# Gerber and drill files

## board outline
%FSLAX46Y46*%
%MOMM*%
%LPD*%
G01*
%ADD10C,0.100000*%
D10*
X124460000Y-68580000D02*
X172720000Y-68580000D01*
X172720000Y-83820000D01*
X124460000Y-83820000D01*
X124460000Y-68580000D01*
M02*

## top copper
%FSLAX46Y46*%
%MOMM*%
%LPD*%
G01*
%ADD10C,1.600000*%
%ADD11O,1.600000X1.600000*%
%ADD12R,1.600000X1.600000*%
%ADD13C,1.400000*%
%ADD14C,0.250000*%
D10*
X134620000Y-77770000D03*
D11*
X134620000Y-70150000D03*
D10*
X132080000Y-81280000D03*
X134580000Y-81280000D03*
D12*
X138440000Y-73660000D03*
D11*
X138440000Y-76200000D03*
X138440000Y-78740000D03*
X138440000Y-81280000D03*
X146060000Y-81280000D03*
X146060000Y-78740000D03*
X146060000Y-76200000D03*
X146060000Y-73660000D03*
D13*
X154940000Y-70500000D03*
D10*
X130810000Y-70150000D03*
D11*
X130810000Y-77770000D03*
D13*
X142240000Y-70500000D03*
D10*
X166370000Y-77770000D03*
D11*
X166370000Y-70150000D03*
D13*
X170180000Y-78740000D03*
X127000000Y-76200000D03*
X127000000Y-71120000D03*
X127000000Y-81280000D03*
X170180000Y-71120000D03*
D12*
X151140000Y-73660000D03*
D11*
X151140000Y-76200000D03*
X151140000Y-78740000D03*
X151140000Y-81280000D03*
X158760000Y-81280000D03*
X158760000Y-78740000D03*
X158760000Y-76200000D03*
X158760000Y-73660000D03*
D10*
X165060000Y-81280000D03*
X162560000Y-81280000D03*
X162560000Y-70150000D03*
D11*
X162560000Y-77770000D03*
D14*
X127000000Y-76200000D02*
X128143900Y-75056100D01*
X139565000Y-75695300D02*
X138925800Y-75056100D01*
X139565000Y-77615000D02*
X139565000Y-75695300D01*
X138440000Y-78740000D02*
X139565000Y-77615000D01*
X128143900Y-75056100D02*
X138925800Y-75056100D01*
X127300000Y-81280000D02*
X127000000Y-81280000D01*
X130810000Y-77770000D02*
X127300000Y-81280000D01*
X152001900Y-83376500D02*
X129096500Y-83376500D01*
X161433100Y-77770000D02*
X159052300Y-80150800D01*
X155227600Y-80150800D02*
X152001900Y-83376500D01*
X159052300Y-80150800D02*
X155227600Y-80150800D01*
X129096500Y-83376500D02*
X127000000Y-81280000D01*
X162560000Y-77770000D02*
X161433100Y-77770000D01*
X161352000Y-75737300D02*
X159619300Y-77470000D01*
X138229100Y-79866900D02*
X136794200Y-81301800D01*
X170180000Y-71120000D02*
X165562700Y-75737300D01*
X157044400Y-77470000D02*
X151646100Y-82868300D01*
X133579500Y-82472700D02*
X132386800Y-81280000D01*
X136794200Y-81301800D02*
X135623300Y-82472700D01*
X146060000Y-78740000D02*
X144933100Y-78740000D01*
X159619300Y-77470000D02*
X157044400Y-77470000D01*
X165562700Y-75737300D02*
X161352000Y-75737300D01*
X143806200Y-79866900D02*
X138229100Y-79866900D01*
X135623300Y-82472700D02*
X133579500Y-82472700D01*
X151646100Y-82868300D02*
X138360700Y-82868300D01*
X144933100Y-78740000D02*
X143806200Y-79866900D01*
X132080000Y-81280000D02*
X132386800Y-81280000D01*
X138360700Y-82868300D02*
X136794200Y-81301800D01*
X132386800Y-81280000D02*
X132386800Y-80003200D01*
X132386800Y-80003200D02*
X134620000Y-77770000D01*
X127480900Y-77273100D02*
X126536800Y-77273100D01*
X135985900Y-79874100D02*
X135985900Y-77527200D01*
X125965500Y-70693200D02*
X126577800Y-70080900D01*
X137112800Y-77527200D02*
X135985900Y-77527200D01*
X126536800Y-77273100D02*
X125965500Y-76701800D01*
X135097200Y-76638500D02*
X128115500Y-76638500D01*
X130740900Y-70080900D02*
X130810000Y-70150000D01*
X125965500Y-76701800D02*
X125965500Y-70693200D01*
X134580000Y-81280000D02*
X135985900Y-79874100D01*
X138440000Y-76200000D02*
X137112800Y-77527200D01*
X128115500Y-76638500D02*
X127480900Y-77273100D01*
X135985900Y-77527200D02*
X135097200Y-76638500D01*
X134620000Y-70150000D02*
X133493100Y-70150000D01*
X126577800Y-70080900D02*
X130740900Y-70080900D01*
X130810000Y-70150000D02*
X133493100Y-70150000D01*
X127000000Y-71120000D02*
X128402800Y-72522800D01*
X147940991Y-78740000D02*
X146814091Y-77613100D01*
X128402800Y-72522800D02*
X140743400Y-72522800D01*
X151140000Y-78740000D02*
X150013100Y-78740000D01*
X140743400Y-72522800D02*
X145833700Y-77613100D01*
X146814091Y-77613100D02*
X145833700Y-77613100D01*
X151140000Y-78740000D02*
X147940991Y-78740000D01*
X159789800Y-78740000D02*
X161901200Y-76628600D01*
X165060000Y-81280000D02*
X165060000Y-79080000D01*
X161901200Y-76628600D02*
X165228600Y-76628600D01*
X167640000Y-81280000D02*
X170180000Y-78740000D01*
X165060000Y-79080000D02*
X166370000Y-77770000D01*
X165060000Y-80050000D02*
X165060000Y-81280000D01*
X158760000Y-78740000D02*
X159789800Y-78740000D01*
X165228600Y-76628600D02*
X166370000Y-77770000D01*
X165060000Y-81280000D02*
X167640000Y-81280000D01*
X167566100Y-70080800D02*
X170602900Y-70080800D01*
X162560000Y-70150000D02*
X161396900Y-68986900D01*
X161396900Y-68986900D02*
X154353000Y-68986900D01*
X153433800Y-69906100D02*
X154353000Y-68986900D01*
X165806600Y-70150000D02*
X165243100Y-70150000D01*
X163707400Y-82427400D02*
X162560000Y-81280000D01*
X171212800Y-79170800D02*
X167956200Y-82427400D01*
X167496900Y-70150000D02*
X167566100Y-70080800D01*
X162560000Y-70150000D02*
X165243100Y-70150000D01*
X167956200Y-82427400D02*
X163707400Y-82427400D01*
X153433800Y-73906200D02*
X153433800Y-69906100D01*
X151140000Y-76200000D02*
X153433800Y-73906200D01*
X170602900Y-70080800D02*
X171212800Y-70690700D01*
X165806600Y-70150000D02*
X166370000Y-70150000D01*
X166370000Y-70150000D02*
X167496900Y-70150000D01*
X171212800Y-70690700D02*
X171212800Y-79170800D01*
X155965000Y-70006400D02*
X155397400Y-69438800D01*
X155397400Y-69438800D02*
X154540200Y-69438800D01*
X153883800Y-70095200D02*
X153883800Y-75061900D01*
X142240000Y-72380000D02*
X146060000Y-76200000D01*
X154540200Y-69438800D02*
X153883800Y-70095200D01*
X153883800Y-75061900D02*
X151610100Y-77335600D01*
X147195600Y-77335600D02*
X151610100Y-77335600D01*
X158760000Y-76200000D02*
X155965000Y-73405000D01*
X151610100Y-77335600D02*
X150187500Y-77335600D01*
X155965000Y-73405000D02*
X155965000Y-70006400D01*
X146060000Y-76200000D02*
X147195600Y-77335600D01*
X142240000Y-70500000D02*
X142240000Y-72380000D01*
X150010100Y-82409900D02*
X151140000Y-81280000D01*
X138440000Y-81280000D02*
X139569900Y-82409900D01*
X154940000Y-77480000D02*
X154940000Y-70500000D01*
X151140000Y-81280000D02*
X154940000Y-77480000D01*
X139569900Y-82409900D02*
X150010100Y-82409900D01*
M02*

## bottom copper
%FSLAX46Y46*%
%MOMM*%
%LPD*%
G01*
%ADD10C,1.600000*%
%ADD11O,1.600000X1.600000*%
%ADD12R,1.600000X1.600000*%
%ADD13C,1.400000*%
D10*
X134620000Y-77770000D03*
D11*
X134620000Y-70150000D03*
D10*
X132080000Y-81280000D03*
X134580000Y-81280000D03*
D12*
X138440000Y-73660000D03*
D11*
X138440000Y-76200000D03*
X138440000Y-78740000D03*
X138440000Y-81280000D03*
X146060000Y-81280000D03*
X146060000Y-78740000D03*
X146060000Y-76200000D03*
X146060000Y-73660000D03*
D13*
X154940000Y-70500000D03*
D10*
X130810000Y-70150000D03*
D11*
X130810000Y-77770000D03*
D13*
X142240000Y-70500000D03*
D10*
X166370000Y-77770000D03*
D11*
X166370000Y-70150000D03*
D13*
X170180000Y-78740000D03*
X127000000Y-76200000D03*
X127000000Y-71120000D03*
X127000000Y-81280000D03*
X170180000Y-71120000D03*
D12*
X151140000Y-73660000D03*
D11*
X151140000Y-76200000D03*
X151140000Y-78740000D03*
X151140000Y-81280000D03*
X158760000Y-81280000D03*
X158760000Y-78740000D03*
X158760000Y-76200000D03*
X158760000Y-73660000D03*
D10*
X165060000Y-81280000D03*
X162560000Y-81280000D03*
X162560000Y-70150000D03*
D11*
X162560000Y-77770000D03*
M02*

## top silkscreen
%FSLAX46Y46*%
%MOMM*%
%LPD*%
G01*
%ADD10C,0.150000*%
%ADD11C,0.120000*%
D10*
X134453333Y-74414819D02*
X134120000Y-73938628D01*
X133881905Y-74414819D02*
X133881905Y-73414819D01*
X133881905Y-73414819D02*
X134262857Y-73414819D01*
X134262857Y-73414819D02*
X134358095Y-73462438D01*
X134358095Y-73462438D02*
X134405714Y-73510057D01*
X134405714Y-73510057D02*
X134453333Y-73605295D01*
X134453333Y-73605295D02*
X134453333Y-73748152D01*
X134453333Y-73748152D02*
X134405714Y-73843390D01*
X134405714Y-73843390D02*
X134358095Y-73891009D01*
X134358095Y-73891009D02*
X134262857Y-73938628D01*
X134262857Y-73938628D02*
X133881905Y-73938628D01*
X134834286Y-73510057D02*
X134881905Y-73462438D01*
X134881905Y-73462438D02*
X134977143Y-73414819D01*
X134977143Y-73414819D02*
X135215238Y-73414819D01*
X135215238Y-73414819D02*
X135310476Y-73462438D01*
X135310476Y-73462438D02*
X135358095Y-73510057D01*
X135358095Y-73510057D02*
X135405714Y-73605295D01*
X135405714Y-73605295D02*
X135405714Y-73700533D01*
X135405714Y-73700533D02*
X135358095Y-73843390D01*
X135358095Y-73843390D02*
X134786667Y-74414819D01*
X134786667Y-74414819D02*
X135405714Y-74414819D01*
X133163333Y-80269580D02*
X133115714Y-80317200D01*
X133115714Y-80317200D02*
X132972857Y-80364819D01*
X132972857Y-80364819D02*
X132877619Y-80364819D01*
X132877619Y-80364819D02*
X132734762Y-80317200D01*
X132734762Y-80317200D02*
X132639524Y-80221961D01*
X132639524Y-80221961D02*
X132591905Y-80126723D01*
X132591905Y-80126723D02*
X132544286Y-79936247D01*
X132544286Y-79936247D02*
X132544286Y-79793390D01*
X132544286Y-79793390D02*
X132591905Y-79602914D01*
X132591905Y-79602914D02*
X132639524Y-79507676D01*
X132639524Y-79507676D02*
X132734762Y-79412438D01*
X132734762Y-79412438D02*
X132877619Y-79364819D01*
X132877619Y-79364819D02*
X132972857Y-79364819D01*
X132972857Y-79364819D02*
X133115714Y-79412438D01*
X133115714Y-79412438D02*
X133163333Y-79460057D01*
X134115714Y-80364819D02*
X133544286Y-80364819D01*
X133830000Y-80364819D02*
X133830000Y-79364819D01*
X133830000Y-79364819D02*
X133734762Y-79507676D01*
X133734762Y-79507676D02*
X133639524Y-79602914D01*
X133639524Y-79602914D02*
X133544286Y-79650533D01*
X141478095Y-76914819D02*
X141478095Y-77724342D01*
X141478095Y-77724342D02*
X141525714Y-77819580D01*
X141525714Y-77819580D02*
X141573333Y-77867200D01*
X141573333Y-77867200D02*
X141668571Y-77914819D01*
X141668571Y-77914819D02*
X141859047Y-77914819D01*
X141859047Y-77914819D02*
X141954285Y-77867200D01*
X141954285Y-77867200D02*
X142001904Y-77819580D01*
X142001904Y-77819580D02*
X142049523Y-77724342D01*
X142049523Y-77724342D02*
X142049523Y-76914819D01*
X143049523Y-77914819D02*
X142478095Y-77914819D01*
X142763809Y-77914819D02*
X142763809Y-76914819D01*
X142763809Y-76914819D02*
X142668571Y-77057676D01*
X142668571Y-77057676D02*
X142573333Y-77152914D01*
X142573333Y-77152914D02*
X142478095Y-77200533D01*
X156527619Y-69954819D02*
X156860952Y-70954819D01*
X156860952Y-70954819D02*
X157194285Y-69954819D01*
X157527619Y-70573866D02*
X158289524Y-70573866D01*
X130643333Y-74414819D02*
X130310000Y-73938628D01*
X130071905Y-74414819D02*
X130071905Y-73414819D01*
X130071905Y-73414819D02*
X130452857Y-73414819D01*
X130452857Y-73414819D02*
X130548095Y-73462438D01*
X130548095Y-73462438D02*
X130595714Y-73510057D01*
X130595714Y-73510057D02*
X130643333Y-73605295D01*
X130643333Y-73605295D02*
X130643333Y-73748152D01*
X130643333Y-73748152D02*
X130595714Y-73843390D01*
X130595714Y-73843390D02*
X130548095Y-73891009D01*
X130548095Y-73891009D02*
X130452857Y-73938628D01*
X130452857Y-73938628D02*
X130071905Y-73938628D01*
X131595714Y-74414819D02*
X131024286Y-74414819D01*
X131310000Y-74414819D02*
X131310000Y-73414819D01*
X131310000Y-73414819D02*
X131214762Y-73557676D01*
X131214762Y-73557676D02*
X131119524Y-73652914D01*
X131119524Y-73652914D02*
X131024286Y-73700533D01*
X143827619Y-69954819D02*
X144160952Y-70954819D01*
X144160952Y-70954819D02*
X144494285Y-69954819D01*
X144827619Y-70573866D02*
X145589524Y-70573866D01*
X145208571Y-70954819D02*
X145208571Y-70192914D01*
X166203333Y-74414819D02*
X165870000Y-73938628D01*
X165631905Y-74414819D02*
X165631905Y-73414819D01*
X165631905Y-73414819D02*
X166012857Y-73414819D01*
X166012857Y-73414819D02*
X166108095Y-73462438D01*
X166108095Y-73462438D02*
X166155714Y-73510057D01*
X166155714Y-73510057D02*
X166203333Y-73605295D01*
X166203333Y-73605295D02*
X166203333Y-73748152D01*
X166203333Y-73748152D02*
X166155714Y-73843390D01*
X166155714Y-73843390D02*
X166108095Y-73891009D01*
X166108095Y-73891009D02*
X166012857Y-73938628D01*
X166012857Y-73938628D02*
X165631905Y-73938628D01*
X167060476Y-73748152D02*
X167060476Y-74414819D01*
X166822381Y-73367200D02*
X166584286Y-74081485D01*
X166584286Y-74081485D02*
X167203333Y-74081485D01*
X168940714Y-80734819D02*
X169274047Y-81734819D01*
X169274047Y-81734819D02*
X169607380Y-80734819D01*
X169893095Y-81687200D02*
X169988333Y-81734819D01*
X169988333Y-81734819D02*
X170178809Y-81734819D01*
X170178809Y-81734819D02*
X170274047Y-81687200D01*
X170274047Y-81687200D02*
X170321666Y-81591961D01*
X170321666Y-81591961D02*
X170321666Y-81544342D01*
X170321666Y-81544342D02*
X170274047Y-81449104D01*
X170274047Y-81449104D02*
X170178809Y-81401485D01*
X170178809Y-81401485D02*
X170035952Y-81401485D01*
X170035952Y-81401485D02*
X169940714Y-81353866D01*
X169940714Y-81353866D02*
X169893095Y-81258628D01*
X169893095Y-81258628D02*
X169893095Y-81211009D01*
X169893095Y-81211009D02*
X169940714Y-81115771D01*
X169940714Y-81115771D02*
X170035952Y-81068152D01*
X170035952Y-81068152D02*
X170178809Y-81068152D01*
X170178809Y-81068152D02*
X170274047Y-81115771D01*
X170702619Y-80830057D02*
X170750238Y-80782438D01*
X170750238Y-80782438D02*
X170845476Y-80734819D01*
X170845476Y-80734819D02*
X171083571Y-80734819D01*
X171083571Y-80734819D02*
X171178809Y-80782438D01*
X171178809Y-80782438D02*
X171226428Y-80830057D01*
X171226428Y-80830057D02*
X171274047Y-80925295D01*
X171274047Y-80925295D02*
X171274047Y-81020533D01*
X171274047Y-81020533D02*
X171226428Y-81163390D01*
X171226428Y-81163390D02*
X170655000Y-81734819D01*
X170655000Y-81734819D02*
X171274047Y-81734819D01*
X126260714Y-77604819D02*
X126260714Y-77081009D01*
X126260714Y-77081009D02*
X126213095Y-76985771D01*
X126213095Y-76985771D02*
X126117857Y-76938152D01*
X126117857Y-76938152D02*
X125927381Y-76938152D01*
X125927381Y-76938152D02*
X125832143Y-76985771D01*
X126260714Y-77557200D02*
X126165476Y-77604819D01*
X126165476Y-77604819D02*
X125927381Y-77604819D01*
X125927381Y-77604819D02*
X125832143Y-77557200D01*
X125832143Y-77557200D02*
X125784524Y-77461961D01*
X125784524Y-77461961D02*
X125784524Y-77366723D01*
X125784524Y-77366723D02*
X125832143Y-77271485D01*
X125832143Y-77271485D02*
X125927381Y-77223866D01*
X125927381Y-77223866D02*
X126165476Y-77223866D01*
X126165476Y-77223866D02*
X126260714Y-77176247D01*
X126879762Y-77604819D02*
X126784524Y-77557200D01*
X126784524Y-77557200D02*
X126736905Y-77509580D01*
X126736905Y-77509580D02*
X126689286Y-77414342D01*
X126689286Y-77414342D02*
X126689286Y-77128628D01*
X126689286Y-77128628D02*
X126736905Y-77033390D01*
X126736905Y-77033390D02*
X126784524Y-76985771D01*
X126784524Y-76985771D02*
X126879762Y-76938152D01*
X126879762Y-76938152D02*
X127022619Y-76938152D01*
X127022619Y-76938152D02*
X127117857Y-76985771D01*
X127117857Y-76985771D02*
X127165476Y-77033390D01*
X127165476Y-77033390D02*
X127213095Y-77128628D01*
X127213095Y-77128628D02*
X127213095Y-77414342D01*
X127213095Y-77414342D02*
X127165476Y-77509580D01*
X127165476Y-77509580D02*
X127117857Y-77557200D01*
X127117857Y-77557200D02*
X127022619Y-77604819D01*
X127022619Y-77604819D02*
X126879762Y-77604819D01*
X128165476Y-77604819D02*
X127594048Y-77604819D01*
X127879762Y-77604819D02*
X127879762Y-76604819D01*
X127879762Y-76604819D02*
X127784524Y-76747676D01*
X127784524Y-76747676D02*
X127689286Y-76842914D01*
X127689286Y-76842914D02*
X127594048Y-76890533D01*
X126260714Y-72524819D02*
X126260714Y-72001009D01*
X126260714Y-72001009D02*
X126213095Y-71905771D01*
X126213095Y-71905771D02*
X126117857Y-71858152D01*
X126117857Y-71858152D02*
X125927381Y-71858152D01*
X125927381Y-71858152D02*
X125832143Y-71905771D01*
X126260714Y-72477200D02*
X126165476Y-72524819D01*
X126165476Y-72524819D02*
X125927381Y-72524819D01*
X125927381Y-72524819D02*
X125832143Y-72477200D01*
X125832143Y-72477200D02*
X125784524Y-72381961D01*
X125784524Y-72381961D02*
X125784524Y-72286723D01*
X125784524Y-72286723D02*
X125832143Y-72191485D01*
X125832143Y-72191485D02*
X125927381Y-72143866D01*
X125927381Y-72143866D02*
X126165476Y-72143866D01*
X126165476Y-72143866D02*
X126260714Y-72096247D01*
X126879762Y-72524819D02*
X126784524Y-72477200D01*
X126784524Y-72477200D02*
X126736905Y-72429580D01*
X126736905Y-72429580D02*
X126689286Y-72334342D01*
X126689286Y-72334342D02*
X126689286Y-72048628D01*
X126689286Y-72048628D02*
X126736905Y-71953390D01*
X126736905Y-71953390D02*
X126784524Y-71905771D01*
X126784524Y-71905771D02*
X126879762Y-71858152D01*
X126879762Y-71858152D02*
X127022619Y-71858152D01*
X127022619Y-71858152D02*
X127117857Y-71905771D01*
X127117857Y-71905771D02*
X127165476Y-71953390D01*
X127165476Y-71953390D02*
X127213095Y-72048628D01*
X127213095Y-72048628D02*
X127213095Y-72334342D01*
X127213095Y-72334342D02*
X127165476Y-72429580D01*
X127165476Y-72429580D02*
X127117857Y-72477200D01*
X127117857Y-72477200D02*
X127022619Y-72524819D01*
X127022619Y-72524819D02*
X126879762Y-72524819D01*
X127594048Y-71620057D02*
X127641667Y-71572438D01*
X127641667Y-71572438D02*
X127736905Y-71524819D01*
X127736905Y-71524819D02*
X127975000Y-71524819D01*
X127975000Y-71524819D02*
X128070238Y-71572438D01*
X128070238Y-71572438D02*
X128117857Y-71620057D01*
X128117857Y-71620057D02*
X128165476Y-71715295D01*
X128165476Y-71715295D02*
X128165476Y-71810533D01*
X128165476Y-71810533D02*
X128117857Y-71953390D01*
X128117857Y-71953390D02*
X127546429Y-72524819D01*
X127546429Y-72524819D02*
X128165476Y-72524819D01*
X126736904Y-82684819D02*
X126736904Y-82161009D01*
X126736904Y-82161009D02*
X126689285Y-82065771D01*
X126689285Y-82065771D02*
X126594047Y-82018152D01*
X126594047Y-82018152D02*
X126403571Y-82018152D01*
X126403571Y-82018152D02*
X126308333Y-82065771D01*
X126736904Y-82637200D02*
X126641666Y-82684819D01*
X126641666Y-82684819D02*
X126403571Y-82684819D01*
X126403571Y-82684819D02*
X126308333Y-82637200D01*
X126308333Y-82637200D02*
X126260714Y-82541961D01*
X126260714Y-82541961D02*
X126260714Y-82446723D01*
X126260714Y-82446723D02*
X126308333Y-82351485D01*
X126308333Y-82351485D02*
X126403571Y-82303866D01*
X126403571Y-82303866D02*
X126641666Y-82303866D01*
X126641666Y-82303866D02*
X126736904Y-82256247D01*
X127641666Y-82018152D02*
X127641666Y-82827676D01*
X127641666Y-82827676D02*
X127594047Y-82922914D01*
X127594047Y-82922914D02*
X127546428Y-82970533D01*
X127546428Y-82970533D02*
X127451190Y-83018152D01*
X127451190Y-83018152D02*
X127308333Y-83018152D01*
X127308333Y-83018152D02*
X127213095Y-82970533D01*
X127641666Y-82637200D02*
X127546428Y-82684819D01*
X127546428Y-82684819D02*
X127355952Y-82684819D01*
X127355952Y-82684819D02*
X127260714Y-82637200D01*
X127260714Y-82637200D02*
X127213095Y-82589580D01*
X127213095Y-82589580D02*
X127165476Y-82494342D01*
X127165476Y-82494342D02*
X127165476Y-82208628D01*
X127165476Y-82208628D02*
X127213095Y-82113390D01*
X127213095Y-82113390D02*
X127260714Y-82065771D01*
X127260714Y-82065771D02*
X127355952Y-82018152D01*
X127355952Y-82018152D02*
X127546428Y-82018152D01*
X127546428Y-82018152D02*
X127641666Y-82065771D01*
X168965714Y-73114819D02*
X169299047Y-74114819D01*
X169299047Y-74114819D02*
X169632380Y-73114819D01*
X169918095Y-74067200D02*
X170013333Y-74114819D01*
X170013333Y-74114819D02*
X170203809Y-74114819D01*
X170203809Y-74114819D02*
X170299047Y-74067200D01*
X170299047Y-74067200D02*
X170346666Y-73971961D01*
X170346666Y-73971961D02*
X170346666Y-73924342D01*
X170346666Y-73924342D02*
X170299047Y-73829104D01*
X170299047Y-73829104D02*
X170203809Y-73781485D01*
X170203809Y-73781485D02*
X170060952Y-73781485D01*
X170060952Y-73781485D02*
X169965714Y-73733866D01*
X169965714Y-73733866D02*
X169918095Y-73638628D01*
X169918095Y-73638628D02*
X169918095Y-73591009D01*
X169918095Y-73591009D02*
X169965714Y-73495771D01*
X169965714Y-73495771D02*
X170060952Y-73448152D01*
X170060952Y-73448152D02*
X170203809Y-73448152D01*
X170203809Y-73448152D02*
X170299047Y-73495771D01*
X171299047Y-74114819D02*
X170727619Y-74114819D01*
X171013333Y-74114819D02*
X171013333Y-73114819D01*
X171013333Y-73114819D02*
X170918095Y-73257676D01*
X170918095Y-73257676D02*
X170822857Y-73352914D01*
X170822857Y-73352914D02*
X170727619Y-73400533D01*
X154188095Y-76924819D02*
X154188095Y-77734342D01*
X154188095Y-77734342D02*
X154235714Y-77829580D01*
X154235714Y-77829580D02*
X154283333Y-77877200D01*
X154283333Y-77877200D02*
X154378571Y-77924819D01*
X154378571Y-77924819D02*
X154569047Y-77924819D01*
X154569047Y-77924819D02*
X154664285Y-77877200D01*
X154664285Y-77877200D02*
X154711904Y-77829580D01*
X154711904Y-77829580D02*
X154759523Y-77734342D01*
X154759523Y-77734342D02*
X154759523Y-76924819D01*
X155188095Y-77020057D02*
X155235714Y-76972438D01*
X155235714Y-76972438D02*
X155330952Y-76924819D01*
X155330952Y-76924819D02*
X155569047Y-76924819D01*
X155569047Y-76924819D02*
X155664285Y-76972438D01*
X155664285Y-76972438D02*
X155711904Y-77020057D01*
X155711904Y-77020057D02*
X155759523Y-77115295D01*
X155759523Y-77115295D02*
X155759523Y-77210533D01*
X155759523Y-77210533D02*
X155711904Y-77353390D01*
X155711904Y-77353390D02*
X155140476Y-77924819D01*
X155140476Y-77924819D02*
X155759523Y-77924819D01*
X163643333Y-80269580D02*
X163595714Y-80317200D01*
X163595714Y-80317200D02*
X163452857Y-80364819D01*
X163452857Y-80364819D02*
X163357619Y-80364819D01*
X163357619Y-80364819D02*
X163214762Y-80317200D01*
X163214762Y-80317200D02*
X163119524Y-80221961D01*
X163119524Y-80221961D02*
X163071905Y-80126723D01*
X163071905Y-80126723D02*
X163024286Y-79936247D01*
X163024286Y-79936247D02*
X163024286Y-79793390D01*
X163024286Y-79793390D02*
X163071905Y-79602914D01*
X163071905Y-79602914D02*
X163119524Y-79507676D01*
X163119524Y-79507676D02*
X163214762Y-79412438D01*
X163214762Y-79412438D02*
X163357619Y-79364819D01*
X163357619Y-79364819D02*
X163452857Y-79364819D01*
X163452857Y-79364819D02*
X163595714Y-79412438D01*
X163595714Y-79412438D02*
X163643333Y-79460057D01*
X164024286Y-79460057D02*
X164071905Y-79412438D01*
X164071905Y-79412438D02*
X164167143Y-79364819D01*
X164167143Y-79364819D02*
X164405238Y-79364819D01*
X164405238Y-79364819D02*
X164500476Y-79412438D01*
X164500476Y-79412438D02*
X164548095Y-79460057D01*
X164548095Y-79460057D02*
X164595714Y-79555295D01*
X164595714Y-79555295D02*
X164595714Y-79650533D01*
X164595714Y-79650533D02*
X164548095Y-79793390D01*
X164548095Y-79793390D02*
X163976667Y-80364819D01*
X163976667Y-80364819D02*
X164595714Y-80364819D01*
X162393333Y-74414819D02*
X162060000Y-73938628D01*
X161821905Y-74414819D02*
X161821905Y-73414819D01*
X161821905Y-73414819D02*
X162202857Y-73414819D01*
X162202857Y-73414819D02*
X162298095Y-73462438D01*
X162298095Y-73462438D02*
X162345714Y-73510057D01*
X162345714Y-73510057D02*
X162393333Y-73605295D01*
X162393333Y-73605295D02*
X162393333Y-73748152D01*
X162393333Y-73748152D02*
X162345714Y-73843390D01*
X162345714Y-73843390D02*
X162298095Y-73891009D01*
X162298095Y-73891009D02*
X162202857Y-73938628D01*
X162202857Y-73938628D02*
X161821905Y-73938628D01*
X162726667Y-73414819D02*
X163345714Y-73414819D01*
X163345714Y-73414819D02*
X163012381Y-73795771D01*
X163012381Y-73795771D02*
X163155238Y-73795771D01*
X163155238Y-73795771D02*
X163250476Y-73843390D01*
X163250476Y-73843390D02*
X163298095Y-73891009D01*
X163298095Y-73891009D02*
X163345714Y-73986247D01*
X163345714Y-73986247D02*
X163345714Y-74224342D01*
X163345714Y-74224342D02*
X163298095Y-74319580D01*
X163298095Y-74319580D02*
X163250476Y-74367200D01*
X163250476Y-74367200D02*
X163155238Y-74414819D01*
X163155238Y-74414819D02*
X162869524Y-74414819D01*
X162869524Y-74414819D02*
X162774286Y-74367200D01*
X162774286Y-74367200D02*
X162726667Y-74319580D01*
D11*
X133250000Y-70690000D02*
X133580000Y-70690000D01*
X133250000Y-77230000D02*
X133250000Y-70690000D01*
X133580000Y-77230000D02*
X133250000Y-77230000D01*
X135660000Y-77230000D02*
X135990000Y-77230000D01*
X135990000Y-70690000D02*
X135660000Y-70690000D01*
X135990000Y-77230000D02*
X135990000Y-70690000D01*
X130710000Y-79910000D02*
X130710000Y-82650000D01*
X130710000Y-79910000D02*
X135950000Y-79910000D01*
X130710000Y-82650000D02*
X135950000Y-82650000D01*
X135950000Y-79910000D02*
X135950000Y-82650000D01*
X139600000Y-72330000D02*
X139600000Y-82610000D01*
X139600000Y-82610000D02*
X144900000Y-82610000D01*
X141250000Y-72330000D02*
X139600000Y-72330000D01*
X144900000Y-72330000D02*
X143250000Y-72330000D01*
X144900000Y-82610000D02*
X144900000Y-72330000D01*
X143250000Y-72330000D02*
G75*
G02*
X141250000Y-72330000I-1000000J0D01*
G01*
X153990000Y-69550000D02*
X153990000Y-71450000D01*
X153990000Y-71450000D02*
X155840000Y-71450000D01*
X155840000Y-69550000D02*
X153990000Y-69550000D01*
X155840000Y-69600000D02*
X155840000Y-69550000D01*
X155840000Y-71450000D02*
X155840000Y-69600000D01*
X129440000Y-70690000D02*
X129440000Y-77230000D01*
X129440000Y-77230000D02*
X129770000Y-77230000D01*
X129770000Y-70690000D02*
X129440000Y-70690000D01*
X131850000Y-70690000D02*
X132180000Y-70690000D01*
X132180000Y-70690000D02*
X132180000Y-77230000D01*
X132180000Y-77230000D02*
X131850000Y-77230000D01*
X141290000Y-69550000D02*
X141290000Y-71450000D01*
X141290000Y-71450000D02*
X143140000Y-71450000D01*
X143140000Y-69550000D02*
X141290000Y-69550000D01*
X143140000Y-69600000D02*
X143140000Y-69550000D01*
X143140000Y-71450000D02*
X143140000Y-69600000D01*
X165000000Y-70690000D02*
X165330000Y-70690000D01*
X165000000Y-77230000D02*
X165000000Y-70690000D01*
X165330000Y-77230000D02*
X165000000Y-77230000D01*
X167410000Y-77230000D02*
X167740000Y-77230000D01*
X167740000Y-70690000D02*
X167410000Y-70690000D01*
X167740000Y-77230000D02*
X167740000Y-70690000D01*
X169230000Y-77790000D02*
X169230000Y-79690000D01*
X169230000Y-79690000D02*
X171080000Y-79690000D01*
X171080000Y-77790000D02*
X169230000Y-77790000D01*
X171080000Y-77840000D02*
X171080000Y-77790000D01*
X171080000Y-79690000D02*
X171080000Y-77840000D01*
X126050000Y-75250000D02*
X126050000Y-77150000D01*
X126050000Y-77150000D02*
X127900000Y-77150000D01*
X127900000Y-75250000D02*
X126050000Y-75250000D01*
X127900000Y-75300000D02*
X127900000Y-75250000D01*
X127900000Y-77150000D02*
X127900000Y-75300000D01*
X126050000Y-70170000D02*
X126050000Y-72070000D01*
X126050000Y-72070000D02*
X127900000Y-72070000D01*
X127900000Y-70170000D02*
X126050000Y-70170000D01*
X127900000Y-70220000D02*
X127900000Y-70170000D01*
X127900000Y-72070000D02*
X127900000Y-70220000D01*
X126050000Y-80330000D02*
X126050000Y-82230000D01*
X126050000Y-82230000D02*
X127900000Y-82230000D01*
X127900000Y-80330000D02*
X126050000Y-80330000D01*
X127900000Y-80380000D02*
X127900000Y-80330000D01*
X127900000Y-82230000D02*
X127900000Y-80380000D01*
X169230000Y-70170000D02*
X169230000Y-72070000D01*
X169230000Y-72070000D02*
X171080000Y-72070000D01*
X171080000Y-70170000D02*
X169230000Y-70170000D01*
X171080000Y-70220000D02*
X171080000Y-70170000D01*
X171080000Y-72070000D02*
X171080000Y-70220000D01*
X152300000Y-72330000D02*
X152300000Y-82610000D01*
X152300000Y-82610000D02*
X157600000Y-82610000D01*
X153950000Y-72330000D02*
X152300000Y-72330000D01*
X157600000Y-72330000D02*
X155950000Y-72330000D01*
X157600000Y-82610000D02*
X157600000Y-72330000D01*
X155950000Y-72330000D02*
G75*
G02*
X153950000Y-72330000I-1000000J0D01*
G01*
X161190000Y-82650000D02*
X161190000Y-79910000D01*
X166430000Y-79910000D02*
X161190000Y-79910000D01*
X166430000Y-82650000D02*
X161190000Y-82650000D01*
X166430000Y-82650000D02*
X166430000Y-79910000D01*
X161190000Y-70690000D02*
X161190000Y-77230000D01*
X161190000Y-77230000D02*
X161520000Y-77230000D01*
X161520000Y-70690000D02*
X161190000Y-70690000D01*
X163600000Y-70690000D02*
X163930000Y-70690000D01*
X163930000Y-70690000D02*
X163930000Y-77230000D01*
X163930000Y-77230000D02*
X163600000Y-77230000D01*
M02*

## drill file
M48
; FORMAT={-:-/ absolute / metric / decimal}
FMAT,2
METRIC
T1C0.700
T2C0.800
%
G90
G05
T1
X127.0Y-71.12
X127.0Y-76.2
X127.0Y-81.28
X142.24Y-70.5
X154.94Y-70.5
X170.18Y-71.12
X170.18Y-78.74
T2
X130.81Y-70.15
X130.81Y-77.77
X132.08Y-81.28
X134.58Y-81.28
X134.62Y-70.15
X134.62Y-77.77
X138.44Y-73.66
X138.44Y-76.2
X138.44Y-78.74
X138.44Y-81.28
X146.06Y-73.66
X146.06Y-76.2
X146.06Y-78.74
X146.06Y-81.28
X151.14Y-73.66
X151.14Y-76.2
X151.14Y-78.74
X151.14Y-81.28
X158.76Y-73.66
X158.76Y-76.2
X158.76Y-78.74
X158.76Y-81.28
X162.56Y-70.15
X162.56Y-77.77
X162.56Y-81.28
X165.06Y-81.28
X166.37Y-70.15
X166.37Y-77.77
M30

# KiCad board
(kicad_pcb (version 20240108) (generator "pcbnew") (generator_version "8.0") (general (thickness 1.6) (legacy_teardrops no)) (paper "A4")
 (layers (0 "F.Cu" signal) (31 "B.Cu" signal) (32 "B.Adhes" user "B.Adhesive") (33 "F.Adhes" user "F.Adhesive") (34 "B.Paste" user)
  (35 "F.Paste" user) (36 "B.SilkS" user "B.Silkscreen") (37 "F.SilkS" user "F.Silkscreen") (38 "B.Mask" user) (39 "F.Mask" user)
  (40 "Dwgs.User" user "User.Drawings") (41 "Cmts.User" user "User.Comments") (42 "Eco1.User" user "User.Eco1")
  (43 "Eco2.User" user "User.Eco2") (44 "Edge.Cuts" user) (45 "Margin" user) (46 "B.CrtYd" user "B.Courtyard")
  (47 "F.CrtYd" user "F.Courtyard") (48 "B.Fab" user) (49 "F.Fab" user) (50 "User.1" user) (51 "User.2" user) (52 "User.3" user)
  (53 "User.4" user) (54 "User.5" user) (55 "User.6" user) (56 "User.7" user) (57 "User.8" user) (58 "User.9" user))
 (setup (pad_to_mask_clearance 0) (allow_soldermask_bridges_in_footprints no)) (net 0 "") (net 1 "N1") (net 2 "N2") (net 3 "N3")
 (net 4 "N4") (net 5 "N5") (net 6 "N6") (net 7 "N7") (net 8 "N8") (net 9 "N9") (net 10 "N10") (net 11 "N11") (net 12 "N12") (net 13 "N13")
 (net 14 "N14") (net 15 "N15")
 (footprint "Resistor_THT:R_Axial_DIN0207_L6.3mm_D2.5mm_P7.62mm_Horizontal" (layer "F.Cu") (at 134.62 77.77 90)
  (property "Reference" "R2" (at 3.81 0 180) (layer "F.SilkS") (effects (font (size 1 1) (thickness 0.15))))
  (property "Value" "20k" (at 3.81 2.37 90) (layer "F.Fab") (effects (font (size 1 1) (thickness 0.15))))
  (fp_line (start 7.08 -1.37) (end 7.08 -1.04) (stroke (width 0.12) (type solid)) (layer "F.SilkS"))
  (fp_line (start 0.54 -1.37) (end 7.08 -1.37) (stroke (width 0.12) (type solid)) (layer "F.SilkS"))
  (fp_line (start 0.54 -1.04) (end 0.54 -1.37) (stroke (width 0.12) (type solid)) (layer "F.SilkS"))
  (fp_line (start 0.54 1.04) (end 0.54 1.37) (stroke (width 0.12) (type solid)) (layer "F.SilkS"))
  (fp_line (start 7.08 1.37) (end 7.08 1.04) (stroke (width 0.12) (type solid)) (layer "F.SilkS"))
  (fp_line (start 0.54 1.37) (end 7.08 1.37) (stroke (width 0.12) (type solid)) (layer "F.SilkS"))
  (pad "1" thru_hole circle (at 0 0 90) (size 1.6 1.6) (drill 0.8) (layers "*.Cu" "*.Mask") (remove_unused_layers no) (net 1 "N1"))
  (pad "2" thru_hole oval (at 7.62 0 90) (size 1.6 1.6) (drill 0.8) (layers "*.Cu" "*.Mask") (remove_unused_layers no) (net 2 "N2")))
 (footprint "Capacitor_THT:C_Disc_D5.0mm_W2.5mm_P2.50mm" (layer "F.Cu") (at 132.08 81.28)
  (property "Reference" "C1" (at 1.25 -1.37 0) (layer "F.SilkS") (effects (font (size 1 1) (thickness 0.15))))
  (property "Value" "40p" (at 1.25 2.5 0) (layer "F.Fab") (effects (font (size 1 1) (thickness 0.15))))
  (fp_line (start -1.37 -1.37) (end -1.37 1.37) (stroke (width 0.12) (type solid)) (layer "F.SilkS"))
  (fp_line (start -1.37 -1.37) (end 3.87 -1.37) (stroke (width 0.12) (type solid)) (layer "F.SilkS"))
  (fp_line (start -1.37 1.37) (end 3.87 1.37) (stroke (width 0.12) (type solid)) (layer "F.SilkS"))
  (fp_line (start 3.87 -1.37) (end 3.87 1.37) (stroke (width 0.12) (type solid)) (layer "F.SilkS"))
  (pad "1" thru_hole circle (at 0 0) (size 1.6 1.6) (drill 0.8) (layers "*.Cu" "*.Mask") (remove_unused_layers no) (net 1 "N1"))
  (pad "2" thru_hole circle (at 2.5 0) (size 1.6 1.6) (drill 0.8) (layers "*.Cu" "*.Mask") (remove_unused_layers no) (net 2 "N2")))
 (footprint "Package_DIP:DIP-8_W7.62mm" (layer "F.Cu") (at 138.44 73.66)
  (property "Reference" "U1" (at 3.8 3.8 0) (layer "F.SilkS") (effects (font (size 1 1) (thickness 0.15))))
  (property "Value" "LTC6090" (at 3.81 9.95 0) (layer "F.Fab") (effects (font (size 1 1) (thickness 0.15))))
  (fp_line (start 1.16 -1.33) (end 1.16 8.95) (stroke (width 0.12) (type solid)) (layer "F.SilkS"))
  (fp_line (start 1.16 8.95) (end 6.46 8.95) (stroke (width 0.12) (type solid)) (layer "F.SilkS"))
  (fp_line (start 2.81 -1.33) (end 1.16 -1.33) (stroke (width 0.12) (type solid)) (layer "F.SilkS"))
  (fp_line (start 6.46 -1.33) (end 4.81 -1.33) (stroke (width 0.12) (type solid)) (layer "F.SilkS"))
  (fp_line (start 6.46 8.95) (end 6.46 -1.33) (stroke (width 0.12) (type solid)) (layer "F.SilkS"))
  (fp_arc (start 4.81 -1.33) (mid 3.81 -0.33) (end 2.81 -1.33) (stroke (width 0.12) (type solid)) (layer "F.SilkS"))
  (pad "1" thru_hole rect (at 0 0) (size 1.6 1.6) (drill 0.8) (layers "*.Cu" "*.Mask") (remove_unused_layers no) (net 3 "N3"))
  (pad "2" thru_hole oval (at 0 2.54) (size 1.6 1.6) (drill 0.8) (layers "*.Cu" "*.Mask") (remove_unused_layers no) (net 2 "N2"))
  (pad "3" thru_hole oval (at 0 5.08) (size 1.6 1.6) (drill 0.8) (layers "*.Cu" "*.Mask") (remove_unused_layers no) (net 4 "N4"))
  (pad "4" thru_hole oval (at 0 7.62) (size 1.6 1.6) (drill 0.8) (layers "*.Cu" "*.Mask") (remove_unused_layers no) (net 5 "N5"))
  (pad "5" thru_hole oval (at 7.62 7.62) (size 1.6 1.6) (drill 0.8) (layers "*.Cu" "*.Mask") (remove_unused_layers no) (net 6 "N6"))
  (pad "6" thru_hole oval (at 7.62 5.08) (size 1.6 1.6) (drill 0.8) (layers "*.Cu" "*.Mask") (remove_unused_layers no) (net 1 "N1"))
  (pad "7" thru_hole oval (at 7.62 2.54) (size 1.6 1.6) (drill 0.8) (layers "*.Cu" "*.Mask") (remove_unused_layers no) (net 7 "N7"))
  (pad "8" thru_hole oval (at 7.62 0) (size 1.6 1.6) (drill 0.8) (layers "*.Cu" "*.Mask") (remove_unused_layers no) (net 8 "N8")))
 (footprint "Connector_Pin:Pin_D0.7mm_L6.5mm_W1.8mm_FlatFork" (layer "F.Cu") (at 154.94 70.5)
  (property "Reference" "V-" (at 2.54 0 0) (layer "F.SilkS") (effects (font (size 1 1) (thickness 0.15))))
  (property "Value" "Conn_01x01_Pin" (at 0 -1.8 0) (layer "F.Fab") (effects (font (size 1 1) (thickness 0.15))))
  (fp_line (start -0.95 -0.95) (end -0.95 0.95) (stroke (width 0.12) (type solid)) (layer "F.SilkS"))
  (fp_line (start -0.95 0.95) (end 0.9 0.95) (stroke (width 0.12) (type solid)) (layer "F.SilkS"))
  (fp_line (start 0.9 -0.95) (end -0.95 -0.95) (stroke (width 0.12) (type solid)) (layer "F.SilkS"))
  (fp_line (start 0.9 -0.9) (end 0.9 -0.95) (stroke (width 0.12) (type solid)) (layer "F.SilkS"))
  (fp_line (start 0.9 0.95) (end 0.9 -0.9) (stroke (width 0.12) (type solid)) (layer "F.SilkS"))
  (pad "1" thru_hole circle (at 0 0) (size 1.4 1.4) (drill 0.7) (layers "*.Cu" "*.Mask") (remove_unused_layers no) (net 5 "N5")))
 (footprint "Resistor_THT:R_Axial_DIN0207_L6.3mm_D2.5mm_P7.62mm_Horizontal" (layer "F.Cu") (at 130.81 70.15 -90)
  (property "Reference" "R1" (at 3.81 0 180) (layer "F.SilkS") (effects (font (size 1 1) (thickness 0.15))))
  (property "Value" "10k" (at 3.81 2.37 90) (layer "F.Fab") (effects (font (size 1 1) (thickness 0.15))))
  (fp_line (start 0.54 1.37) (end 7.08 1.37) (stroke (width 0.12) (type solid)) (layer "F.SilkS"))
  (fp_line (start 7.08 1.37) (end 7.08 1.04) (stroke (width 0.12) (type solid)) (layer "F.SilkS"))
  (fp_line (start 0.54 1.04) (end 0.54 1.37) (stroke (width 0.12) (type solid)) (layer "F.SilkS"))
  (fp_line (start 0.54 -1.04) (end 0.54 -1.37) (stroke (width 0.12) (type solid)) (layer "F.SilkS"))
  (fp_line (start 0.54 -1.37) (end 7.08 -1.37) (stroke (width 0.12) (type solid)) (layer "F.SilkS"))
  (fp_line (start 7.08 -1.37) (end 7.08 -1.04) (stroke (width 0.12) (type solid)) (layer "F.SilkS"))
  (pad "1" thru_hole circle (at 0 0 270) (size 1.6 1.6) (drill 0.8) (layers "*.Cu" "*.Mask") (remove_unused_layers no) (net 2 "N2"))
  (pad "2" thru_hole oval (at 7.62 0 270) (size 1.6 1.6) (drill 0.8) (layers "*.Cu" "*.Mask") (remove_unused_layers no) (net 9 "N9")))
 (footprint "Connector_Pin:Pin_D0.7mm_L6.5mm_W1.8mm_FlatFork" (layer "F.Cu") (at 142.24 70.5)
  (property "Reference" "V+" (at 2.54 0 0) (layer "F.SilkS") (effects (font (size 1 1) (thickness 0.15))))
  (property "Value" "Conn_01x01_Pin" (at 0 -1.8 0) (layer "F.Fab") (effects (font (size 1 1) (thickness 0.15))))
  (fp_line (start -0.95 -0.95) (end -0.95 0.95) (stroke (width 0.12) (type solid)) (layer "F.SilkS"))
  (fp_line (start -0.95 0.95) (end 0.9 0.95) (stroke (width 0.12) (type solid)) (layer "F.SilkS"))
  (fp_line (start 0.9 -0.95) (end -0.95 -0.95) (stroke (width 0.12) (type solid)) (layer "F.SilkS"))
  (fp_line (start 0.9 -0.9) (end 0.9 -0.95) (stroke (width 0.12) (type solid)) (layer "F.SilkS"))
  (fp_line (start 0.9 0.95) (end 0.9 -0.9) (stroke (width 0.12) (type solid)) (layer "F.SilkS"))
  (pad "1" thru_hole circle (at 0 0) (size 1.4 1.4) (drill 0.7) (layers "*.Cu" "*.Mask") (remove_unused_layers no) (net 7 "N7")))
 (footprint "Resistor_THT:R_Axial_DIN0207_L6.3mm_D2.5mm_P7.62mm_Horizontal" (layer "F.Cu") (at 166.37 77.77 90)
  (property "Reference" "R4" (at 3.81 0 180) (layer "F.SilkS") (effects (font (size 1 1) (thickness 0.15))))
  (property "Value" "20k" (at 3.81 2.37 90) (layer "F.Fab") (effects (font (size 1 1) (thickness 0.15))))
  (fp_line (start 7.08 -1.37) (end 7.08 -1.04) (stroke (width 0.12) (type solid)) (layer "F.SilkS"))
  (fp_line (start 0.54 -1.37) (end 7.08 -1.37) (stroke (width 0.12) (type solid)) (layer "F.SilkS"))
  (fp_line (start 0.54 -1.04) (end 0.54 -1.37) (stroke (width 0.12) (type solid)) (layer "F.SilkS"))
  (fp_line (start 0.54 1.04) (end 0.54 1.37) (stroke (width 0.12) (type solid)) (layer "F.SilkS"))
  (fp_line (start 7.08 1.37) (end 7.08 1.04) (stroke (width 0.12) (type solid)) (layer "F.SilkS"))
  (fp_line (start 0.54 1.37) (end 7.08 1.37) (stroke (width 0.12) (type solid)) (layer "F.SilkS"))
  (pad "1" thru_hole circle (at 0 0 90) (size 1.6 1.6) (drill 0.8) (layers "*.Cu" "*.Mask") (remove_unused_layers no) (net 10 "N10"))
  (pad "2" thru_hole oval (at 7.62 0 90) (size 1.6 1.6) (drill 0.8) (layers "*.Cu" "*.Mask") (remove_unused_layers no) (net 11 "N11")))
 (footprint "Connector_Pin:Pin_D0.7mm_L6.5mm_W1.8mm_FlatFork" (layer "F.Cu") (at 170.18 78.74)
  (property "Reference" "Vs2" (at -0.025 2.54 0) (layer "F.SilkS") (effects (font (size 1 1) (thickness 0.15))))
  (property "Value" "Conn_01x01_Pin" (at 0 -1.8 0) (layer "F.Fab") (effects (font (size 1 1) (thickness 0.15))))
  (fp_line (start -0.95 -0.95) (end -0.95 0.95) (stroke (width 0.12) (type solid)) (layer "F.SilkS"))
  (fp_line (start -0.95 0.95) (end 0.9 0.95) (stroke (width 0.12) (type solid)) (layer "F.SilkS"))
  (fp_line (start 0.9 -0.95) (end -0.95 -0.95) (stroke (width 0.12) (type solid)) (layer "F.SilkS"))
  (fp_line (start 0.9 -0.9) (end 0.9 -0.95) (stroke (width 0.12) (type solid)) (layer "F.SilkS"))
  (fp_line (start 0.9 0.95) (end 0.9 -0.9) (stroke (width 0.12) (type solid)) (layer "F.SilkS"))
  (pad "1" thru_hole circle (at 0 0) (size 1.4 1.4) (drill 0.7) (layers "*.Cu" "*.Mask") (remove_unused_layers no) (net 10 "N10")))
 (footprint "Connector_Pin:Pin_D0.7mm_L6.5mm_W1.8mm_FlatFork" (layer "F.Cu") (at 127 76.2)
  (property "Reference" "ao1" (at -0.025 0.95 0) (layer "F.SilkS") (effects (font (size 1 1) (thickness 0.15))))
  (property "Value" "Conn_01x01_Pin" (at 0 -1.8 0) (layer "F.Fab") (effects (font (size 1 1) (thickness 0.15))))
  (fp_line (start -0.95 -0.95) (end -0.95 0.95) (stroke (width 0.12) (type solid)) (layer "F.SilkS"))
  (fp_line (start -0.95 0.95) (end 0.9 0.95) (stroke (width 0.12) (type solid)) (layer "F.SilkS"))
  (fp_line (start 0.9 -0.95) (end -0.95 -0.95) (stroke (width 0.12) (type solid)) (layer "F.SilkS"))
  (fp_line (start 0.9 -0.9) (end 0.9 -0.95) (stroke (width 0.12) (type solid)) (layer "F.SilkS"))
  (fp_line (start 0.9 0.95) (end 0.9 -0.9) (stroke (width 0.12) (type solid)) (layer "F.SilkS"))
  (pad "1" thru_hole circle (at 0 0) (size 1.4 1.4) (drill 0.7) (layers "*.Cu" "*.Mask") (remove_unused_layers no) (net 4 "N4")))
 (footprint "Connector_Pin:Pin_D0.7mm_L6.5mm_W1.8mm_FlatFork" (layer "F.Cu") (at 127 71.12)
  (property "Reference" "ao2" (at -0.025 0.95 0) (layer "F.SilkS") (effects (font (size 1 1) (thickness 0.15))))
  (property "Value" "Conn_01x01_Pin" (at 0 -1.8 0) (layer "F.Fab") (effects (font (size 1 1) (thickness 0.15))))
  (fp_line (start -0.95 -0.95) (end -0.95 0.95) (stroke (width 0.12) (type solid)) (layer "F.SilkS"))
  (fp_line (start -0.95 0.95) (end 0.9 0.95) (stroke (width 0.12) (type solid)) (layer "F.SilkS"))
  (fp_line (start 0.9 -0.95) (end -0.95 -0.95) (stroke (width 0.12) (type solid)) (layer "F.SilkS"))
  (fp_line (start 0.9 -0.9) (end 0.9 -0.95) (stroke (width 0.12) (type solid)) (layer "F.SilkS"))
  (fp_line (start 0.9 0.95) (end 0.9 -0.9) (stroke (width 0.12) (type solid)) (layer "F.SilkS"))
  (pad "1" thru_hole circle (at 0 0) (size 1.4 1.4) (drill 0.7) (layers "*.Cu" "*.Mask") (remove_unused_layers no) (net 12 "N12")))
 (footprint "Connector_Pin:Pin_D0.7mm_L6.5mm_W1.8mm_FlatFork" (layer "F.Cu") (at 127 81.28)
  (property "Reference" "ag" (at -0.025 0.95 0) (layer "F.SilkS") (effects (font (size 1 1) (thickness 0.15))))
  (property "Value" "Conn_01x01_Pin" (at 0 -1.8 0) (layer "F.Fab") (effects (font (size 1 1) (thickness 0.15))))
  (fp_line (start -0.95 -0.95) (end -0.95 0.95) (stroke (width 0.12) (type solid)) (layer "F.SilkS"))
  (fp_line (start -0.95 0.95) (end 0.9 0.95) (stroke (width 0.12) (type solid)) (layer "F.SilkS"))
  (fp_line (start 0.9 -0.95) (end -0.95 -0.95) (stroke (width 0.12) (type solid)) (layer "F.SilkS"))
  (fp_line (start 0.9 -0.9) (end 0.9 -0.95) (stroke (width 0.12) (type solid)) (layer "F.SilkS"))
  (fp_line (start 0.9 0.95) (end 0.9 -0.9) (stroke (width 0.12) (type solid)) (layer "F.SilkS"))
  (pad "1" thru_hole circle (at 0 0) (size 1.4 1.4) (drill 0.7) (layers "*.Cu" "*.Mask") (remove_unused_layers no) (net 9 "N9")))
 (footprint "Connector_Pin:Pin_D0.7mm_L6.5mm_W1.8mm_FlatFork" (layer "F.Cu") (at 170.18 71.12)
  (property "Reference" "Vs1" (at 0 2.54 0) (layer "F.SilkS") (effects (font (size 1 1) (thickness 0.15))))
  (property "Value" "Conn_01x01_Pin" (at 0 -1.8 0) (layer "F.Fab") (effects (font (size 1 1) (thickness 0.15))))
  (fp_line (start -0.95 -0.95) (end -0.95 0.95) (stroke (width 0.12) (type solid)) (layer "F.SilkS"))
  (fp_line (start -0.95 0.95) (end 0.9 0.95) (stroke (width 0.12) (type solid)) (layer "F.SilkS"))
  (fp_line (start 0.9 -0.95) (end -0.95 -0.95) (stroke (width 0.12) (type solid)) (layer "F.SilkS"))
  (fp_line (start 0.9 -0.9) (end 0.9 -0.95) (stroke (width 0.12) (type solid)) (layer "F.SilkS"))
  (fp_line (start 0.9 0.95) (end 0.9 -0.9) (stroke (width 0.12) (type solid)) (layer "F.SilkS"))
  (pad "1" thru_hole circle (at 0 0) (size 1.4 1.4) (drill 0.7) (layers "*.Cu" "*.Mask") (remove_unused_layers no) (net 1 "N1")))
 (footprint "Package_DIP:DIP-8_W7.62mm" (layer "F.Cu") (at 151.14 73.66)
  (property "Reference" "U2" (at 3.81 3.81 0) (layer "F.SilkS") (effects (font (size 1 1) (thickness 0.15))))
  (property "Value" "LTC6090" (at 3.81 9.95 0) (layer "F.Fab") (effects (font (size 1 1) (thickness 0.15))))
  (fp_line (start 1.16 -1.33) (end 1.16 8.95) (stroke (width 0.12) (type solid)) (layer "F.SilkS"))
  (fp_line (start 1.16 8.95) (end 6.46 8.95) (stroke (width 0.12) (type solid)) (layer "F.SilkS"))
  (fp_line (start 2.81 -1.33) (end 1.16 -1.33) (stroke (width 0.12) (type solid)) (layer "F.SilkS"))
  (fp_line (start 6.46 -1.33) (end 4.81 -1.33) (stroke (width 0.12) (type solid)) (layer "F.SilkS"))
  (fp_line (start 6.46 8.95) (end 6.46 -1.33) (stroke (width 0.12) (type solid)) (layer "F.SilkS"))
  (fp_arc (start 4.81 -1.33) (mid 3.81 -0.33) (end 2.81 -1.33) (stroke (width 0.12) (type solid)) (layer "F.SilkS"))
  (pad "1" thru_hole rect (at 0 0) (size 1.6 1.6) (drill 0.8) (layers "*.Cu" "*.Mask") (remove_unused_layers no) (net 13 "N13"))
  (pad "2" thru_hole oval (at 0 2.54) (size 1.6 1.6) (drill 0.8) (layers "*.Cu" "*.Mask") (remove_unused_layers no) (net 11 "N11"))
  (pad "3" thru_hole oval (at 0 5.08) (size 1.6 1.6) (drill 0.8) (layers "*.Cu" "*.Mask") (remove_unused_layers no) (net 12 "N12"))
  (pad "4" thru_hole oval (at 0 7.62) (size 1.6 1.6) (drill 0.8) (layers "*.Cu" "*.Mask") (remove_unused_layers no) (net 5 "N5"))
  (pad "5" thru_hole oval (at 7.62 7.62) (size 1.6 1.6) (drill 0.8) (layers "*.Cu" "*.Mask") (remove_unused_layers no) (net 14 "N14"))
  (pad "6" thru_hole oval (at 7.62 5.08) (size 1.6 1.6) (drill 0.8) (layers "*.Cu" "*.Mask") (remove_unused_layers no) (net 10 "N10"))
  (pad "7" thru_hole oval (at 7.62 2.54) (size 1.6 1.6) (drill 0.8) (layers "*.Cu" "*.Mask") (remove_unused_layers no) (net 7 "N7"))
  (pad "8" thru_hole oval (at 7.62 0) (size 1.6 1.6) (drill 0.8) (layers "*.Cu" "*.Mask") (remove_unused_layers no) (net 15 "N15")))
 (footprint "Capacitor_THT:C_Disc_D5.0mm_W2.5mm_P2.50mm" (layer "F.Cu") (at 165.06 81.28 180)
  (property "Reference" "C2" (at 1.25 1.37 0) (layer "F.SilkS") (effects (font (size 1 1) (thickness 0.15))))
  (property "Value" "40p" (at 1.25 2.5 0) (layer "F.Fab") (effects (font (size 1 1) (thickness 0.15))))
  (fp_line (start 3.87 -1.37) (end 3.87 1.37) (stroke (width 0.12) (type solid)) (layer "F.SilkS"))
  (fp_line (start -1.37 1.37) (end 3.87 1.37) (stroke (width 0.12) (type solid)) (layer "F.SilkS"))
  (fp_line (start -1.37 -1.37) (end 3.87 -1.37) (stroke (width 0.12) (type solid)) (layer "F.SilkS"))
  (fp_line (start -1.37 -1.37) (end -1.37 1.37) (stroke (width 0.12) (type solid)) (layer "F.SilkS"))
  (pad "1" thru_hole circle (at 0 0 180) (size 1.6 1.6) (drill 0.8) (layers "*.Cu" "*.Mask") (remove_unused_layers no) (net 10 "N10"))
  (pad "2" thru_hole circle (at 2.5 0 180) (size 1.6 1.6) (drill 0.8) (layers "*.Cu" "*.Mask") (remove_unused_layers no) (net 11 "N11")))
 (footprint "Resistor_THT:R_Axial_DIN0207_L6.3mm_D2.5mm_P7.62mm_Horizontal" (layer "F.Cu") (at 162.56 70.15 -90)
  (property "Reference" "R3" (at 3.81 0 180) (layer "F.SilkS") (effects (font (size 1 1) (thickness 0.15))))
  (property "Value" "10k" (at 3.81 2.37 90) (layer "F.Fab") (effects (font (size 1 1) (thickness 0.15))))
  (fp_line (start 0.54 1.37) (end 7.08 1.37) (stroke (width 0.12) (type solid)) (layer "F.SilkS"))
  (fp_line (start 7.08 1.37) (end 7.08 1.04) (stroke (width 0.12) (type solid)) (layer "F.SilkS"))
  (fp_line (start 0.54 1.04) (end 0.54 1.37) (stroke (width 0.12) (type solid)) (layer "F.SilkS"))
  (fp_line (start 0.54 -1.04) (end 0.54 -1.37) (stroke (width 0.12) (type solid)) (layer "F.SilkS"))
  (fp_line (start 0.54 -1.37) (end 7.08 -1.37) (stroke (width 0.12) (type solid)) (layer "F.SilkS"))
  (fp_line (start 7.08 -1.37) (end 7.08 -1.04) (stroke (width 0.12) (type solid)) (layer "F.SilkS"))
  (pad "1" thru_hole circle (at 0 0 270) (size 1.6 1.6) (drill 0.8) (layers "*.Cu" "*.Mask") (remove_unused_layers no) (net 11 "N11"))
  (pad "2" thru_hole oval (at 7.62 0 270) (size 1.6 1.6) (drill 0.8) (layers "*.Cu" "*.Mask") (remove_unused_layers no) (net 9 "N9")))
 (gr_rect (start 124.46 68.58) (end 172.72 83.82) (stroke (width 0.1) (type default)) (fill none) (layer "Edge.Cuts"))
 (segment (start 127 76.2) (end 128.1439 75.0561) (width 0.25) (layer "F.Cu") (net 4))
 (segment (start 139.565 75.6953) (end 138.9258 75.0561) (width 0.25) (layer "F.Cu") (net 4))
 (segment (start 139.565 77.615) (end 139.565 75.6953) (width 0.25) (layer "F.Cu") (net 4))
 (segment (start 138.44 78.74) (end 139.565 77.615) (width 0.25) (layer "F.Cu") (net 4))
 (segment (start 128.1439 75.0561) (end 138.9258 75.0561) (width 0.25) (layer "F.Cu") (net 4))
 (segment (start 127.3 81.28) (end 127 81.28) (width 0.25) (layer "F.Cu") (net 9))
 (segment (start 130.81 77.77) (end 127.3 81.28) (width 0.25) (layer "F.Cu") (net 9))
 (segment (start 152.0019 83.3765) (end 129.0965 83.3765) (width 0.25) (layer "F.Cu") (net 9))
 (segment (start 161.4331 77.77) (end 159.0523 80.1508) (width 0.25) (layer "F.Cu") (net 9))
 (segment (start 155.2276 80.1508) (end 152.0019 83.3765) (width 0.25) (layer "F.Cu") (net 9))
 (segment (start 159.0523 80.1508) (end 155.2276 80.1508) (width 0.25) (layer "F.Cu") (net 9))
 (segment (start 129.0965 83.3765) (end 127 81.28) (width 0.25) (layer "F.Cu") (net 9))
 (segment (start 162.56 77.77) (end 161.4331 77.77) (width 0.25) (layer "F.Cu") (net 9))
 (segment (start 161.352 75.7373) (end 159.6193 77.47) (width 0.25) (layer "F.Cu") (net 1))
 (segment (start 138.2291 79.8669) (end 136.7942 81.3018) (width 0.25) (layer "F.Cu") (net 1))
 (segment (start 170.18 71.12) (end 165.5627 75.7373) (width 0.25) (layer "F.Cu") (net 1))
 (segment (start 157.0444 77.47) (end 151.6461 82.8683) (width 0.25) (layer "F.Cu") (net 1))
 (segment (start 133.5795 82.4727) (end 132.3868 81.28) (width 0.25) (layer "F.Cu") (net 1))
 (segment (start 136.7942 81.3018) (end 135.6233 82.4727) (width 0.25) (layer "F.Cu") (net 1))
 (segment (start 146.06 78.74) (end 144.9331 78.74) (width 0.25) (layer "F.Cu") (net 1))
 (segment (start 159.6193 77.47) (end 157.0444 77.47) (width 0.25) (layer "F.Cu") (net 1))
 (segment (start 165.5627 75.7373) (end 161.352 75.7373) (width 0.25) (layer "F.Cu") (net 1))
 (segment (start 143.8062 79.8669) (end 138.2291 79.8669) (width 0.25) (layer "F.Cu") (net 1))
 (segment (start 135.6233 82.4727) (end 133.5795 82.4727) (width 0.25) (layer "F.Cu") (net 1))
 (segment (start 151.6461 82.8683) (end 138.3607 82.8683) (width 0.25) (layer "F.Cu") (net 1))
 (segment (start 144.9331 78.74) (end 143.8062 79.8669) (width 0.25) (layer "F.Cu") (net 1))
 (segment (start 132.08 81.28) (end 132.3868 81.28) (width 0.25) (layer "F.Cu") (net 1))
 (segment (start 138.3607 82.8683) (end 136.7942 81.3018) (width 0.25) (layer "F.Cu") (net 1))
 (segment (start 132.3868 81.28) (end 132.3868 80.0032) (width 0.25) (layer "F.Cu") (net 1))
 (segment (start 132.3868 80.0032) (end 134.62 77.77) (width 0.25) (layer "F.Cu") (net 1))
 (segment (start 127.4809 77.2731) (end 126.5368 77.2731) (width 0.25) (layer "F.Cu") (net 2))
 (segment (start 135.9859 79.8741) (end 135.9859 77.5272) (width 0.25) (layer "F.Cu") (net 2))
 (segment (start 125.9655 70.6932) (end 126.5778 70.0809) (width 0.25) (layer "F.Cu") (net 2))
 (segment (start 137.1128 77.5272) (end 135.9859 77.5272) (width 0.25) (layer "F.Cu") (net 2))
 (segment (start 126.5368 77.2731) (end 125.9655 76.7018) (width 0.25) (layer "F.Cu") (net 2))
 (segment (start 135.0972 76.6385) (end 128.1155 76.6385) (width 0.25) (layer "F.Cu") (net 2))
 (segment (start 130.7409 70.0809) (end 130.81 70.15) (width 0.25) (layer "F.Cu") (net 2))
 (segment (start 125.9655 76.7018) (end 125.9655 70.6932) (width 0.25) (layer "F.Cu") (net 2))
 (segment (start 134.58 81.28) (end 135.9859 79.8741) (width 0.25) (layer "F.Cu") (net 2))
 (segment (start 138.44 76.2) (end 137.1128 77.5272) (width 0.25) (layer "F.Cu") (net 2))
 (segment (start 128.1155 76.6385) (end 127.4809 77.2731) (width 0.25) (layer "F.Cu") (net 2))
 (segment (start 135.9859 77.5272) (end 135.0972 76.6385) (width 0.25) (layer "F.Cu") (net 2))
 (segment (start 134.62 70.15) (end 133.4931 70.15) (width 0.25) (layer "F.Cu") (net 2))
 (segment (start 126.5778 70.0809) (end 130.7409 70.0809) (width 0.25) (layer "F.Cu") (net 2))
 (segment (start 130.81 70.15) (end 133.4931 70.15) (width 0.25) (layer "F.Cu") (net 2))
 (segment (start 127 71.12) (end 128.4028 72.5228) (width 0.25) (layer "F.Cu") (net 12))
 (segment (start 147.940991 78.74) (end 146.814091 77.6131) (width 0.25) (layer "F.Cu") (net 12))
 (segment (start 128.4028 72.5228) (end 140.7434 72.5228) (width 0.25) (layer "F.Cu") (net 12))
 (segment (start 151.14 78.74) (end 150.0131 78.74) (width 0.25) (layer "F.Cu") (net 12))
 (segment (start 140.7434 72.5228) (end 145.8337 77.6131) (width 0.25) (layer "F.Cu") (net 12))
 (segment (start 146.814091 77.6131) (end 145.8337 77.6131) (width 0.25) (layer "F.Cu") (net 12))
 (segment (start 151.14 78.74) (end 147.940991 78.74) (width 0.25) (layer "F.Cu") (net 12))
 (segment (start 159.7898 78.74) (end 161.9012 76.6286) (width 0.25) (layer "F.Cu") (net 10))
 (segment (start 165.06 81.28) (end 165.06 79.08) (width 0.25) (layer "F.Cu") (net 10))
 (segment (start 161.9012 76.6286) (end 165.2286 76.6286) (width 0.25) (layer "F.Cu") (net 10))
 (segment (start 167.64 81.28) (end 170.18 78.74) (width 0.25) (layer "F.Cu") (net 10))
 (segment (start 165.06 79.08) (end 166.37 77.77) (width 0.25) (layer "F.Cu") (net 10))
 (segment (start 165.06 80.05) (end 165.06 81.28) (width 0.25) (layer "F.Cu") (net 10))
 (segment (start 158.76 78.74) (end 159.7898 78.74) (width 0.25) (layer "F.Cu") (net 10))
 (segment (start 165.2286 76.6286) (end 166.37 77.77) (width 0.25) (layer "F.Cu") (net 10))
 (segment (start 165.06 81.28) (end 167.64 81.28) (width 0.25) (layer "F.Cu") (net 10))
 (segment (start 167.5661 70.0808) (end 170.6029 70.0808) (width 0.25) (layer "F.Cu") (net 11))
 (segment (start 162.56 70.15) (end 161.3969 68.9869) (width 0.25) (layer "F.Cu") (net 11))
 (segment (start 161.3969 68.9869) (end 154.353 68.9869) (width 0.25) (layer "F.Cu") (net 11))
 (segment (start 153.4338 69.9061) (end 154.353 68.9869) (width 0.25) (layer "F.Cu") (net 11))
 (segment (start 165.8066 70.15) (end 165.2431 70.15) (width 0.25) (layer "F.Cu") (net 11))
 (segment (start 163.7074 82.4274) (end 162.56 81.28) (width 0.25) (layer "F.Cu") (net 11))
 (segment (start 171.2128 79.1708) (end 167.9562 82.4274) (width 0.25) (layer "F.Cu") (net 11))
 (segment (start 167.4969 70.15) (end 167.5661 70.0808) (width 0.25) (layer "F.Cu") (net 11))
 (segment (start 162.56 70.15) (end 165.2431 70.15) (width 0.25) (layer "F.Cu") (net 11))
 (segment (start 167.9562 82.4274) (end 163.7074 82.4274) (width 0.25) (layer "F.Cu") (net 11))
 (segment (start 153.4338 73.9062) (end 153.4338 69.9061) (width 0.25) (layer "F.Cu") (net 11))
 (segment (start 151.14 76.2) (end 153.4338 73.9062) (width 0.25) (layer "F.Cu") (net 11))
 (segment (start 170.6029 70.0808) (end 171.2128 70.6907) (width 0.25) (layer "F.Cu") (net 11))
 (segment (start 165.8066 70.15) (end 166.37 70.15) (width 0.25) (layer "F.Cu") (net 11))
 (segment (start 166.37 70.15) (end 167.4969 70.15) (width 0.25) (layer "F.Cu") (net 11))
 (segment (start 171.2128 70.6907) (end 171.2128 79.1708) (width 0.25) (layer "F.Cu") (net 11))
 (segment (start 155.965 70.0064) (end 155.3974 69.4388) (width 0.25) (layer "F.Cu") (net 7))
 (segment (start 155.3974 69.4388) (end 154.5402 69.4388) (width 0.25) (layer "F.Cu") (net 7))
 (segment (start 153.8838 70.0952) (end 153.8838 75.0619) (width 0.25) (layer "F.Cu") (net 7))
 (segment (start 142.24 72.38) (end 146.06 76.2) (width 0.25) (layer "F.Cu") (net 7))
 (segment (start 154.5402 69.4388) (end 153.8838 70.0952) (width 0.25) (layer "F.Cu") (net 7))
 (segment (start 153.8838 75.0619) (end 151.6101 77.3356) (width 0.25) (layer "F.Cu") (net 7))
 (segment (start 147.1956 77.3356) (end 151.6101 77.3356) (width 0.25) (layer "F.Cu") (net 7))
 (segment (start 158.76 76.2) (end 155.965 73.405) (width 0.25) (layer "F.Cu") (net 7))
 (segment (start 151.6101 77.3356) (end 150.1875 77.3356) (width 0.25) (layer "F.Cu") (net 7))
 (segment (start 155.965 73.405) (end 155.965 70.0064) (width 0.25) (layer "F.Cu") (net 7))
 (segment (start 146.06 76.2) (end 147.1956 77.3356) (width 0.25) (layer "F.Cu") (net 7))
 (segment (start 142.24 70.5) (end 142.24 72.38) (width 0.25) (layer "F.Cu") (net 7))
 (segment (start 150.0101 82.4099) (end 151.14 81.28) (width 0.25) (layer "F.Cu") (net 5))
 (segment (start 138.44 81.28) (end 139.5699 82.4099) (width 0.25) (layer "F.Cu") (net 5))
 (segment (start 154.94 77.48) (end 154.94 70.5) (width 0.25) (layer "F.Cu") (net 5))
 (segment (start 151.14 81.28) (end 154.94 77.48) (width 0.25) (layer "F.Cu") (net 5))
 (segment (start 139.5699 82.4099) (end 150.0101 82.4099) (width 0.25) (layer "F.Cu") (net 5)))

